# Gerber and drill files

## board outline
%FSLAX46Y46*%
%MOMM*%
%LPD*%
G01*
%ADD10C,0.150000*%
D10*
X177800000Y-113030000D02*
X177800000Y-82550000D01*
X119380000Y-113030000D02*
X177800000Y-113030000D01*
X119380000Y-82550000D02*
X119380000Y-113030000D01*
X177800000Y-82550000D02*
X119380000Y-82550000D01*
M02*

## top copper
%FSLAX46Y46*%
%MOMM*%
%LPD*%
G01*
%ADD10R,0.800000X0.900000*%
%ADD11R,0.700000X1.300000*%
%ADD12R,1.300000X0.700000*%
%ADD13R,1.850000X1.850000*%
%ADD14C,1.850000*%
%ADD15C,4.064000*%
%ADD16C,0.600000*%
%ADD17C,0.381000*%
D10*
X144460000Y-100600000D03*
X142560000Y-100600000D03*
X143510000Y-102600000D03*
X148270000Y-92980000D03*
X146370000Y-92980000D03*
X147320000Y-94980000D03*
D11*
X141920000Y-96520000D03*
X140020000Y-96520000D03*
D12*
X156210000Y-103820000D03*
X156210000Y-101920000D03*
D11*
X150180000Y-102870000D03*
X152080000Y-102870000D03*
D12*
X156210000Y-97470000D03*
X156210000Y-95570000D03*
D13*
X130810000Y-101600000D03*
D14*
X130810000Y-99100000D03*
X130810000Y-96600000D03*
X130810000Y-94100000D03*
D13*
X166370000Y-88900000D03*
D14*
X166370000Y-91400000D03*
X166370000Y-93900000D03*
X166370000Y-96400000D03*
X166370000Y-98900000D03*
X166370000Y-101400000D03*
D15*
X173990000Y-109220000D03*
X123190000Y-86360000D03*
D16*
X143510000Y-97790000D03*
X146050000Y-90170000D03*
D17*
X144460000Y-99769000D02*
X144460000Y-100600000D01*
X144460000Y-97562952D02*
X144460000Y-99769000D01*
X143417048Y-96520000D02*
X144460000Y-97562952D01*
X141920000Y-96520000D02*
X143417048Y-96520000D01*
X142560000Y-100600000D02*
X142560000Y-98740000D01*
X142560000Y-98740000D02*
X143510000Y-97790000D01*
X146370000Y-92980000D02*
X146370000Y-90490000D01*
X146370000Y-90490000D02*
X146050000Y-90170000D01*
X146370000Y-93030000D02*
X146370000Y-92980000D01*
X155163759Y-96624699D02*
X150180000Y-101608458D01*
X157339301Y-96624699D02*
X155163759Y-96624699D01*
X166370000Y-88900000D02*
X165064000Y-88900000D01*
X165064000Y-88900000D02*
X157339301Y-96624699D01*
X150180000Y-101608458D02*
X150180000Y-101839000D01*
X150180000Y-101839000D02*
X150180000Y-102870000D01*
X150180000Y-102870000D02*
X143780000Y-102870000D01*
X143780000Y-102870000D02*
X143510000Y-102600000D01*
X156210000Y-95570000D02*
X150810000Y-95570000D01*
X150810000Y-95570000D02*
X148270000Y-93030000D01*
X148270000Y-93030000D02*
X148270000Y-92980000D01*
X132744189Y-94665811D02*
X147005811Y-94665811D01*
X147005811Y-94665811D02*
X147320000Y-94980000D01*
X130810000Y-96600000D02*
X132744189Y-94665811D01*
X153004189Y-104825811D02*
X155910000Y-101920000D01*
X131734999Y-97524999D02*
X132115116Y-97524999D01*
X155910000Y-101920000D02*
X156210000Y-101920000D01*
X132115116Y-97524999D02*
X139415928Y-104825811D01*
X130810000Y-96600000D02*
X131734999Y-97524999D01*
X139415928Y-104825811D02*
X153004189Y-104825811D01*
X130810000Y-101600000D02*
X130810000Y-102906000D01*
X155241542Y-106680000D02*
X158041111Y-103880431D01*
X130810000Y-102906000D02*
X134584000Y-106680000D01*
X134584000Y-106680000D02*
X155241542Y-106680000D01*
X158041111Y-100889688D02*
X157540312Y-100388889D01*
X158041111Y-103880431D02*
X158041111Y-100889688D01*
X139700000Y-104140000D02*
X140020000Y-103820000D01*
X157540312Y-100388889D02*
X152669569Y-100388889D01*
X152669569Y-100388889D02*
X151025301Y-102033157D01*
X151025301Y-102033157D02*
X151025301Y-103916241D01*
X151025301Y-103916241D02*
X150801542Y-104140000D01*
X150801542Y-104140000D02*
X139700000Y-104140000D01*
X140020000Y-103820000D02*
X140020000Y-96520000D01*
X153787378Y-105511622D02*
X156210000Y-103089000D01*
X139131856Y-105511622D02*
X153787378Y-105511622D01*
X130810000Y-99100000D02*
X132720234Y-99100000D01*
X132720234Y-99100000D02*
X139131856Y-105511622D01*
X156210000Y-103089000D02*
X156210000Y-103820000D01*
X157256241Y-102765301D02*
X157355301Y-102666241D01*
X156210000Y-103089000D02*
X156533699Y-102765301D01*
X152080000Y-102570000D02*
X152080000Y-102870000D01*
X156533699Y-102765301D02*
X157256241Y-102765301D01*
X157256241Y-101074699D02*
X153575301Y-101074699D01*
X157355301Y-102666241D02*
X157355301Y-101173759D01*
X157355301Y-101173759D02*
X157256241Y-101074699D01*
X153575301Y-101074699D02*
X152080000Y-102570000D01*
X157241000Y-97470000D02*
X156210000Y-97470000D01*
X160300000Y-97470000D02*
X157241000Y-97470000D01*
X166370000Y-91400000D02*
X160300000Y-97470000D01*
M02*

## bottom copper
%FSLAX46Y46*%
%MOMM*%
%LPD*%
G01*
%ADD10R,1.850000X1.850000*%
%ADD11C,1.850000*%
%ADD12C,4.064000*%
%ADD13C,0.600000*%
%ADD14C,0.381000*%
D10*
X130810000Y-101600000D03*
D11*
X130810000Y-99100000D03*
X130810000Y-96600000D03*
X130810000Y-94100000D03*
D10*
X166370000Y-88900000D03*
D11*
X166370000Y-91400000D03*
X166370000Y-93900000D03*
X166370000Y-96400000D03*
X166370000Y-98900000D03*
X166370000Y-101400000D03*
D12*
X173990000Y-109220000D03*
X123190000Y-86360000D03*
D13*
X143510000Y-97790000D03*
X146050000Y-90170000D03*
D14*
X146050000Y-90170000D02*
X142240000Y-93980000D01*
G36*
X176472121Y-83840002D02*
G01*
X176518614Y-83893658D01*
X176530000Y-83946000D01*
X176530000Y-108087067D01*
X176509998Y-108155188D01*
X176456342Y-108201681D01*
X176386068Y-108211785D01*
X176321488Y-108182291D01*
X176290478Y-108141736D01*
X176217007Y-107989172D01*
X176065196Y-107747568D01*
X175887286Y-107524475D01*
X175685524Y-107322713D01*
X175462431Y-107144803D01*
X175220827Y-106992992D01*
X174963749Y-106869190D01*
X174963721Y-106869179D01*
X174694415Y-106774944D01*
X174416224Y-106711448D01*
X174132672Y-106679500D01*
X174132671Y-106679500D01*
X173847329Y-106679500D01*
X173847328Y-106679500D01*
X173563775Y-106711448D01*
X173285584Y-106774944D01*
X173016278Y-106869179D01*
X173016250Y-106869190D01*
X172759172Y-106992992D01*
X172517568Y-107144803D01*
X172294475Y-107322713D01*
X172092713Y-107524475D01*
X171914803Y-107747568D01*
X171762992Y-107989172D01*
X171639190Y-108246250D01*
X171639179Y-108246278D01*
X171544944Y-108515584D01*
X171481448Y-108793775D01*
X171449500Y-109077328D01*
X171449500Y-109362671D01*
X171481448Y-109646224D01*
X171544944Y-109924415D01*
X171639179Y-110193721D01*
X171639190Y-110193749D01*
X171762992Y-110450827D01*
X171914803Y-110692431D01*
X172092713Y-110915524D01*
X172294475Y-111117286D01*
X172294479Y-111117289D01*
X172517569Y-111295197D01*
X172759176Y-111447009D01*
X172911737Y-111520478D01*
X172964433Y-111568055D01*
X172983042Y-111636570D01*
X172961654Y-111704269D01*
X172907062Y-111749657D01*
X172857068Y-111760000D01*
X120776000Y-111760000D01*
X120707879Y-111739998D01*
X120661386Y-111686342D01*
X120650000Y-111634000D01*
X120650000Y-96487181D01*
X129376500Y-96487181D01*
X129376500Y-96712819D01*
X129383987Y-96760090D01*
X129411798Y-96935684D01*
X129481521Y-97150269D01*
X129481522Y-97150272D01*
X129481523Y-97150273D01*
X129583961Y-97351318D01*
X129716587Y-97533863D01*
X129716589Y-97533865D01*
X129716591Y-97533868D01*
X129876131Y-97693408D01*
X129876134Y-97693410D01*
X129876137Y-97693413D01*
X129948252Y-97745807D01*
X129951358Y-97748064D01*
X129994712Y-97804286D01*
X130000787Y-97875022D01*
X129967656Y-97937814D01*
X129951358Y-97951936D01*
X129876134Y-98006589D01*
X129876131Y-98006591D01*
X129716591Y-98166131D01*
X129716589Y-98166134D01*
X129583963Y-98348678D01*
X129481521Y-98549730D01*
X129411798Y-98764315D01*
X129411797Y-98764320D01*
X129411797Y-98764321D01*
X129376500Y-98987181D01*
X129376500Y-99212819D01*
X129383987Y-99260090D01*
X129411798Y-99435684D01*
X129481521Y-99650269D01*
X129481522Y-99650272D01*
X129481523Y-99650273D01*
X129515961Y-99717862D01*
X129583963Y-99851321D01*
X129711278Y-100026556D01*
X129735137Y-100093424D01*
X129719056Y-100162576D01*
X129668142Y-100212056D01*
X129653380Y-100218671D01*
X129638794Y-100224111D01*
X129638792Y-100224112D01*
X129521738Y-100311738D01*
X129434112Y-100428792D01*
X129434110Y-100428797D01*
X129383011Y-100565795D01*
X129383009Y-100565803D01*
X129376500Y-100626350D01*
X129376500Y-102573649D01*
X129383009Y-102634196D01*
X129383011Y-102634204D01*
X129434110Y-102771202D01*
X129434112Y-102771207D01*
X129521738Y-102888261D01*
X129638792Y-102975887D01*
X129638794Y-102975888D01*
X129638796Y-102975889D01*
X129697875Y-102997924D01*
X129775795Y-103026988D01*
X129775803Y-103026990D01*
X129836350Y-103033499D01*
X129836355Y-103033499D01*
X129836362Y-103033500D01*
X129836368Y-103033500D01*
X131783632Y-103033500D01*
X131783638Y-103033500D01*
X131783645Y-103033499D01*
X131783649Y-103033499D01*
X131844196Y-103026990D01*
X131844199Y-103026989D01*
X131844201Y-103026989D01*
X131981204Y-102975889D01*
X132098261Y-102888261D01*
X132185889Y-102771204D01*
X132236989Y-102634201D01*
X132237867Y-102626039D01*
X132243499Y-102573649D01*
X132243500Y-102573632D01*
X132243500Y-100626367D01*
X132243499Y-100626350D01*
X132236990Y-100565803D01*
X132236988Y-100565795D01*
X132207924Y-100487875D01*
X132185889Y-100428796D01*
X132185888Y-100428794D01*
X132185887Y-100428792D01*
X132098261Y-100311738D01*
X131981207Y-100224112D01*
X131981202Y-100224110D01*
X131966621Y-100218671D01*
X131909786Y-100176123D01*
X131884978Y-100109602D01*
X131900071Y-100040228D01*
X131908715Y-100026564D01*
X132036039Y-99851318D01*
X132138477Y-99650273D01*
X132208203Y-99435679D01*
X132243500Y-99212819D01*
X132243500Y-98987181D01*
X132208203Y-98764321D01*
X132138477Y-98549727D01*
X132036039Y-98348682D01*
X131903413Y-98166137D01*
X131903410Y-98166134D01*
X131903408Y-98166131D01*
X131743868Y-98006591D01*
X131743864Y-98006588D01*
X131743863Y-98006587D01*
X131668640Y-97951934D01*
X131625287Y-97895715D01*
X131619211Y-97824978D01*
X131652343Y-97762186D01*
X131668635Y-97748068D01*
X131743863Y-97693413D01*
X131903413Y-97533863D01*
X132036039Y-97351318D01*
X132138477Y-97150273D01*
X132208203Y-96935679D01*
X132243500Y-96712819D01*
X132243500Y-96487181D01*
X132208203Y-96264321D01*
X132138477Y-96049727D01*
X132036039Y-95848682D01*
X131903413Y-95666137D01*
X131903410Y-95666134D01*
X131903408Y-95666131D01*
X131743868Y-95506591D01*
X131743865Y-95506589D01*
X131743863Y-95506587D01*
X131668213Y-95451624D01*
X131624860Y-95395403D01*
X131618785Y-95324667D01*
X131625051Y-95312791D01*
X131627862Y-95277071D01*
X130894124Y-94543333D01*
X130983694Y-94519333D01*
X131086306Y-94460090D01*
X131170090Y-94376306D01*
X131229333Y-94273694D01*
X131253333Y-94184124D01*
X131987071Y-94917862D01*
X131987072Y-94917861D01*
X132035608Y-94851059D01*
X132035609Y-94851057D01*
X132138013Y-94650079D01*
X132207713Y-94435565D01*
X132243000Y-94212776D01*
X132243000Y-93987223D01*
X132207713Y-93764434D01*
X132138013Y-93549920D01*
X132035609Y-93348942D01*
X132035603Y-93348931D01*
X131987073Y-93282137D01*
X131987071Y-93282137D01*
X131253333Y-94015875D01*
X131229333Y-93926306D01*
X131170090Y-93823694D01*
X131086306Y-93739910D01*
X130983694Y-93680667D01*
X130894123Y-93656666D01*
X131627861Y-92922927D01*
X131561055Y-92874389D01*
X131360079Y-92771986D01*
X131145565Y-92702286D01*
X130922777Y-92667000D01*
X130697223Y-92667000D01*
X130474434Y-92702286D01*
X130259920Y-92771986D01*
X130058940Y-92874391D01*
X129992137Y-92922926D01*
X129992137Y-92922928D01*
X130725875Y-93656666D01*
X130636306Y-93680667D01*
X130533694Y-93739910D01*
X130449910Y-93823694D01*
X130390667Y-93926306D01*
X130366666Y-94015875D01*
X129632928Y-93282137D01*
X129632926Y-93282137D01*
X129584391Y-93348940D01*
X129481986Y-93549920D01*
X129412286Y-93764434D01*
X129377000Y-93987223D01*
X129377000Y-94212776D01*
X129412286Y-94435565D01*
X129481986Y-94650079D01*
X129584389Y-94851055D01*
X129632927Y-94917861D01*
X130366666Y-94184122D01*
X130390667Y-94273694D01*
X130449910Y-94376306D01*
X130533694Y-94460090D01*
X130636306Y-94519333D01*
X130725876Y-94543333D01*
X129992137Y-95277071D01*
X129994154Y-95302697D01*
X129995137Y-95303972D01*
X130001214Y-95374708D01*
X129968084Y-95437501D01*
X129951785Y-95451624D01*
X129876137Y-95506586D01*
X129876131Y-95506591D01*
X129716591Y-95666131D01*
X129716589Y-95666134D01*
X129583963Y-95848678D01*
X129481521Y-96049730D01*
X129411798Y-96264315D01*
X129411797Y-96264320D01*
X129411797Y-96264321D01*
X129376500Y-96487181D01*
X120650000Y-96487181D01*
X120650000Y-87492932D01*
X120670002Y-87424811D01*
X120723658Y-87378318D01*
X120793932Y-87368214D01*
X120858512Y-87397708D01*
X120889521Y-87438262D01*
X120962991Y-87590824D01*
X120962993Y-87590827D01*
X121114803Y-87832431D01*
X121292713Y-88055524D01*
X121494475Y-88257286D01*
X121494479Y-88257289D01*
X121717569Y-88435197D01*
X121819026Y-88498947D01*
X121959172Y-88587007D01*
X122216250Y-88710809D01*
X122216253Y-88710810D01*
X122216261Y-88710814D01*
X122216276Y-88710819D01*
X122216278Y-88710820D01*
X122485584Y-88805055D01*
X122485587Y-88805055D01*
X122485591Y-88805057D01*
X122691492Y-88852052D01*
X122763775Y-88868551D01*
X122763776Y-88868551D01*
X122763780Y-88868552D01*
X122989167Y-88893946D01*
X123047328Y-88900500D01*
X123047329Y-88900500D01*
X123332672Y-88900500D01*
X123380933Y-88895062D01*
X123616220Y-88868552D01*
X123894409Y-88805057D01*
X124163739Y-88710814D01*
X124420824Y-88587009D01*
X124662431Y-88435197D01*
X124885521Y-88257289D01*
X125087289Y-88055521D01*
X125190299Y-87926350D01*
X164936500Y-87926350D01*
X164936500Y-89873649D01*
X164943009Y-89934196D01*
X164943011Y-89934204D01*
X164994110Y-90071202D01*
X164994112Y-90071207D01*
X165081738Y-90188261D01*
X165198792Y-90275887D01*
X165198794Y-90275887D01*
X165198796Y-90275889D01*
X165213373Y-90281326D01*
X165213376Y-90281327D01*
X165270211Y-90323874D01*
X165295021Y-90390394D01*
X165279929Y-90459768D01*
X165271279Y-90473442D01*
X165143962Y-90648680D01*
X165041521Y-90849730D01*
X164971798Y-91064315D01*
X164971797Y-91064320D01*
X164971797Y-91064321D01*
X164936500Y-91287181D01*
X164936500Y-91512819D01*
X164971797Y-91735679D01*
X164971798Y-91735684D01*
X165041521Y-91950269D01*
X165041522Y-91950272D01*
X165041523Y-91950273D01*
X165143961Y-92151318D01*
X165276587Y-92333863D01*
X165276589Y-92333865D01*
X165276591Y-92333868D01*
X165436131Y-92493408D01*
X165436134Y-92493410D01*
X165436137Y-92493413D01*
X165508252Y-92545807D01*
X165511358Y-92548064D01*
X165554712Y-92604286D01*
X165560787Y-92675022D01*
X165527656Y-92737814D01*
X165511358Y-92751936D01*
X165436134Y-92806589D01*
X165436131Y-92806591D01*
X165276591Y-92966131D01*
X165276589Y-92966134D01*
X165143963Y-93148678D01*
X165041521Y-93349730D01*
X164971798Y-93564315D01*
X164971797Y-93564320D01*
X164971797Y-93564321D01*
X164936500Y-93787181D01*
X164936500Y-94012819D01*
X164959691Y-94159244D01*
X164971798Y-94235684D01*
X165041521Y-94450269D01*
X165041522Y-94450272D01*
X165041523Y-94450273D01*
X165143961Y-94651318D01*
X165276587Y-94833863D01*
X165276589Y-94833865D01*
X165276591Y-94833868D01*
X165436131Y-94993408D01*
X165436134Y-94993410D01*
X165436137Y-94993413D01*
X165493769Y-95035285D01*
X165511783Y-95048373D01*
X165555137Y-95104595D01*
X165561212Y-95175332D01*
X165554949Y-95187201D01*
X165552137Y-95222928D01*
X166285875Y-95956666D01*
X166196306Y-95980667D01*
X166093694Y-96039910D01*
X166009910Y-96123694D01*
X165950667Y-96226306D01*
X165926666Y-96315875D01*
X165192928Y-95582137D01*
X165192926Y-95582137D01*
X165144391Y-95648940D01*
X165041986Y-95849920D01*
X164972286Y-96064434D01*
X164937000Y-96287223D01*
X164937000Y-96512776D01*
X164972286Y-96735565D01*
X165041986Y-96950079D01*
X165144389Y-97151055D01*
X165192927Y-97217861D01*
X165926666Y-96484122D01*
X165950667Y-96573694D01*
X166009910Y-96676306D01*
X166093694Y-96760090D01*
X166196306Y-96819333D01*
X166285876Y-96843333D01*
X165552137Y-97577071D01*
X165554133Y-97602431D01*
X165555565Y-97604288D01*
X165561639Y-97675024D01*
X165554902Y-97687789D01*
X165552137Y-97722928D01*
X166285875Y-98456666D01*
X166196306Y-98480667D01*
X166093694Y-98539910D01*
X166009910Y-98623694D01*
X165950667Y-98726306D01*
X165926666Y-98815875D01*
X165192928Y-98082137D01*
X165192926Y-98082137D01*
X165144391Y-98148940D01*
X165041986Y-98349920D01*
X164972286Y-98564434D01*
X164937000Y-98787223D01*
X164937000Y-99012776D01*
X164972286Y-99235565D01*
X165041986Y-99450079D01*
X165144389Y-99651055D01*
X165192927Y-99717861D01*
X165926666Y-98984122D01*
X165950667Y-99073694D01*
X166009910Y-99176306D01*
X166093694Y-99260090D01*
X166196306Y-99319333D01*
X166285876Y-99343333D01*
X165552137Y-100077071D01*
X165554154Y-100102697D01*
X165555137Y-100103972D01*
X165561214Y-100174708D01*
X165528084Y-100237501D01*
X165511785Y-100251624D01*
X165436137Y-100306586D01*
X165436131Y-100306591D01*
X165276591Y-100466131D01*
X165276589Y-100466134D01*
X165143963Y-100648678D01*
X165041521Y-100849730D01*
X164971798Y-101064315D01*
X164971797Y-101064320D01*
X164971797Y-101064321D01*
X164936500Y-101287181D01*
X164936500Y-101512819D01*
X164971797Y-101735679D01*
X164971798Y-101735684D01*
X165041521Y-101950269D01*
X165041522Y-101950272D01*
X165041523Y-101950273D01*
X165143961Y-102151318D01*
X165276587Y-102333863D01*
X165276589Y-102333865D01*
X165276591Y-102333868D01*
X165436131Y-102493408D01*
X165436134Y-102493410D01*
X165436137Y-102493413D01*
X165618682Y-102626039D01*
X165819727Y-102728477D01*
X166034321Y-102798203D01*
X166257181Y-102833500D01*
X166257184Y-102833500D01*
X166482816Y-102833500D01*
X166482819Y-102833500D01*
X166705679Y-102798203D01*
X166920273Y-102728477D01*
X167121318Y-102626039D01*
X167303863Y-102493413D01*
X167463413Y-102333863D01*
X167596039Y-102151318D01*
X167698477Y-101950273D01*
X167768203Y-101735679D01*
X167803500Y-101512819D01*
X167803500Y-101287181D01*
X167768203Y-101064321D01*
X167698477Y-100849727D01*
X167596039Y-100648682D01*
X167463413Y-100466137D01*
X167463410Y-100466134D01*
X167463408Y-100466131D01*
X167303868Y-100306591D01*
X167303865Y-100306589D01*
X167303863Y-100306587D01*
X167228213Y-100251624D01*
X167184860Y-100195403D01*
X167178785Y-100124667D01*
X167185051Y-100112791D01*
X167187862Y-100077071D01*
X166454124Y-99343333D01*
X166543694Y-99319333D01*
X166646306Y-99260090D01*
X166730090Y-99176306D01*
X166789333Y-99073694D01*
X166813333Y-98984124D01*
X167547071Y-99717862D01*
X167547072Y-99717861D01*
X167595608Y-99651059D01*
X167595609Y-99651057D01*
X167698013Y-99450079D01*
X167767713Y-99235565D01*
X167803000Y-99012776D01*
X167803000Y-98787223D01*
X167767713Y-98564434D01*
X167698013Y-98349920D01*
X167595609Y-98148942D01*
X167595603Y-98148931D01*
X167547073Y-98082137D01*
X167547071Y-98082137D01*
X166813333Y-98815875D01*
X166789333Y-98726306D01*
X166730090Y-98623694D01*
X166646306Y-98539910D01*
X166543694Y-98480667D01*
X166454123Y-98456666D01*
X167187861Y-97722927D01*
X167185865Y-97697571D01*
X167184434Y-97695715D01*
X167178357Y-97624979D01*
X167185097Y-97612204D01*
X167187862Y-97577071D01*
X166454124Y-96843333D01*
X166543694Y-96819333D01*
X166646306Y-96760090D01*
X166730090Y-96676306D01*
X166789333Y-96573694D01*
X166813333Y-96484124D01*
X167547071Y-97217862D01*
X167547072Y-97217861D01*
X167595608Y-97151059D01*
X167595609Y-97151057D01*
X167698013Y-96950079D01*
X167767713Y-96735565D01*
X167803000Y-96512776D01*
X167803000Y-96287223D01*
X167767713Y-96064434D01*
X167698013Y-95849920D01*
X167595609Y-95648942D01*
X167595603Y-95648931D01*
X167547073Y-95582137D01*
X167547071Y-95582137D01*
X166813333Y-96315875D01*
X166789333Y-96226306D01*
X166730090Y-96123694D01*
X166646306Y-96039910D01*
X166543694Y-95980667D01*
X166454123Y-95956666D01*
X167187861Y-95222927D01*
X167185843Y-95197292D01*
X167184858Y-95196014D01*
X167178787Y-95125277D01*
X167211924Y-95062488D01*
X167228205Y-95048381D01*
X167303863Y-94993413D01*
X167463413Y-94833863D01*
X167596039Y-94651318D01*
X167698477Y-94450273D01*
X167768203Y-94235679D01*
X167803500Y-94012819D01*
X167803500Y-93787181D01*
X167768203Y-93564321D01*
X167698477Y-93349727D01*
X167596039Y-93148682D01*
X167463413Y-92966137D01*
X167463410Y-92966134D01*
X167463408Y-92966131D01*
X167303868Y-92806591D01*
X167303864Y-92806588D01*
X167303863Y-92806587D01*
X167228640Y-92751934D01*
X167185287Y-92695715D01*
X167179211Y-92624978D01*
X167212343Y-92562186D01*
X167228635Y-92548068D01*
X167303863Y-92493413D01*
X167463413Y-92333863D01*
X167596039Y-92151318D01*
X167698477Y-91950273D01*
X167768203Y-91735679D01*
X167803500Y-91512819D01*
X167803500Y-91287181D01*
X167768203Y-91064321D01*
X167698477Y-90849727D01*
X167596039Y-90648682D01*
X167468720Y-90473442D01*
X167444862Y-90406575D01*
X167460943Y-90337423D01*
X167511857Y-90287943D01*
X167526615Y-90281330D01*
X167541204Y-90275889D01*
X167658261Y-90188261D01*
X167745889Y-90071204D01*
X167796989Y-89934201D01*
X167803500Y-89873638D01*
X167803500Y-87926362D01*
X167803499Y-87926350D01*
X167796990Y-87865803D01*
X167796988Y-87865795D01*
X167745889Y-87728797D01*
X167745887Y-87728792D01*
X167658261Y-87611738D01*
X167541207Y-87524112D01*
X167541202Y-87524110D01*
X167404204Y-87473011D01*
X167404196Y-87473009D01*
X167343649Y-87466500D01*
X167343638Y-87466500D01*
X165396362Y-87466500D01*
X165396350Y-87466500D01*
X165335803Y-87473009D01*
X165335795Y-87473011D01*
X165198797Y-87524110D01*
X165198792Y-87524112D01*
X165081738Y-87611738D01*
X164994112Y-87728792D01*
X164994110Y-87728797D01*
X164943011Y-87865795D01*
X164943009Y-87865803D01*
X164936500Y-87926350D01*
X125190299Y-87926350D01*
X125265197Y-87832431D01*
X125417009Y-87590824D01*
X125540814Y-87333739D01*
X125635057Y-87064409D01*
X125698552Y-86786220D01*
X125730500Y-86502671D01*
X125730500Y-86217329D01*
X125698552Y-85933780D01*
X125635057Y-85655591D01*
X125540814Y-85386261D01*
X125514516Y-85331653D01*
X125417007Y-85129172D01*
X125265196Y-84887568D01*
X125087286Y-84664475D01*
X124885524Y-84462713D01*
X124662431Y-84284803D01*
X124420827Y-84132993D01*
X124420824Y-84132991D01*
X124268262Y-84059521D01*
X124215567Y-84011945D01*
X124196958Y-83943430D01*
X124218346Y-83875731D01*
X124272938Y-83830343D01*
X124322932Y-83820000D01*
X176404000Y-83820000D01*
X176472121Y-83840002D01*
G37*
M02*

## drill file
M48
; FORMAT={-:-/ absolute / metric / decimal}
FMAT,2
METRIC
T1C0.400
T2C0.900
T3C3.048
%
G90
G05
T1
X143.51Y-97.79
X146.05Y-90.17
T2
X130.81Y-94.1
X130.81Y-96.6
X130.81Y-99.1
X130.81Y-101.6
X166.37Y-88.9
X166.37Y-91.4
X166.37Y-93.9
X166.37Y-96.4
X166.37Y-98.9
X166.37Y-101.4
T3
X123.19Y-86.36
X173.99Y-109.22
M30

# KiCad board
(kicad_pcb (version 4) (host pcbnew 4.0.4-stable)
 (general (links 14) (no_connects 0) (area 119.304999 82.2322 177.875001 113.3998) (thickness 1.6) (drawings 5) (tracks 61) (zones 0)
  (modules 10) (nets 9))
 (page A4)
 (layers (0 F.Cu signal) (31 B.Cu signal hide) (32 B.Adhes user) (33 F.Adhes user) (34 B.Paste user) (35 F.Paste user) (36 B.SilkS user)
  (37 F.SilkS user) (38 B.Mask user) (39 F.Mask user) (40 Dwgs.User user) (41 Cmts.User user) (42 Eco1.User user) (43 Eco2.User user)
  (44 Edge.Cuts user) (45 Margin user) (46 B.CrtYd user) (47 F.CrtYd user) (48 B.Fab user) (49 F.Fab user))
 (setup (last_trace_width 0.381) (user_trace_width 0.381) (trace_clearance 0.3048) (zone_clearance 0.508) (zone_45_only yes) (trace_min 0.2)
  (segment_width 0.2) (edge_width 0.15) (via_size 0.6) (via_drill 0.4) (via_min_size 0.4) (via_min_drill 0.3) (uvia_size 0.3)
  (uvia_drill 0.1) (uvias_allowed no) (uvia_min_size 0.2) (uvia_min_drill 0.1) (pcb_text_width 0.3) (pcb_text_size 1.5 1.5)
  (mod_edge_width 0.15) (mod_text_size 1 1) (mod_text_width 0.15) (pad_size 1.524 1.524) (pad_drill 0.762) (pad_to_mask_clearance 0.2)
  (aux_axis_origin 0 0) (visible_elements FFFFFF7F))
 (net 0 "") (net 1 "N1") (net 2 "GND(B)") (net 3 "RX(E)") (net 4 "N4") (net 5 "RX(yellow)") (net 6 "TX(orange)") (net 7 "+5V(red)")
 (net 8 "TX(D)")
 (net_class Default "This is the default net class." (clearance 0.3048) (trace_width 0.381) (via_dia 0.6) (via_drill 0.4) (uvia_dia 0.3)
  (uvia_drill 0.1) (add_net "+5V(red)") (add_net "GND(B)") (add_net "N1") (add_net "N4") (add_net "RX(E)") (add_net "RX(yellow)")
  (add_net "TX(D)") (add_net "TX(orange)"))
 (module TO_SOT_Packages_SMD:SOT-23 (layer F.Cu) (at 143.51 101.6 270)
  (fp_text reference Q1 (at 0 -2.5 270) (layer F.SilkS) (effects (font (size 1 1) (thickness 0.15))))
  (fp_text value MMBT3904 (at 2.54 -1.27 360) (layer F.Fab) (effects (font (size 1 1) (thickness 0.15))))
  (pad 1 smd rect (at -1 -0.95 270) (size 0.9 0.8) (layers F.Cu F.Paste F.Mask) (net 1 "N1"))
  (pad 2 smd rect (at -1 0.95 270) (size 0.9 0.8) (layers F.Cu F.Paste F.Mask) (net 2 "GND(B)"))
  (pad 3 smd rect (at 1 0 270) (size 0.9 0.8) (layers F.Cu F.Paste F.Mask) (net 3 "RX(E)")))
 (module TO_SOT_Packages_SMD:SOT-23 (layer F.Cu) (at 147.32 93.98 270)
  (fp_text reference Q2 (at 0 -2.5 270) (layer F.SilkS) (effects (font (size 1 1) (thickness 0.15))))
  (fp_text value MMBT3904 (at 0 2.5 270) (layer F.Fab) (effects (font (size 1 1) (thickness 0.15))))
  (pad 1 smd rect (at -1 -0.95 270) (size 0.9 0.8) (layers F.Cu F.Paste F.Mask) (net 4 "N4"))
  (pad 2 smd rect (at -1 0.95 270) (size 0.9 0.8) (layers F.Cu F.Paste F.Mask) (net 2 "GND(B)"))
  (pad 3 smd rect (at 1 0 270) (size 0.9 0.8) (layers F.Cu F.Paste F.Mask) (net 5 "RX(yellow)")))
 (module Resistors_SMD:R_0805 (layer F.Cu) (at 140.97 96.52 180)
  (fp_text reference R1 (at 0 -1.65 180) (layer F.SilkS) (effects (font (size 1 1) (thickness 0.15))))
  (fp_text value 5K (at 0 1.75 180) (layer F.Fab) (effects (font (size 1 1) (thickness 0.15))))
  (pad 1 smd rect (at -0.95 0 180) (size 0.7 1.3) (layers F.Cu F.Paste F.Mask) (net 1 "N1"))
  (pad 2 smd rect (at 0.95 0 180) (size 0.7 1.3) (layers F.Cu F.Paste F.Mask) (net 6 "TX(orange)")))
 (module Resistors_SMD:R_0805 (layer F.Cu) (at 156.21 102.87 90)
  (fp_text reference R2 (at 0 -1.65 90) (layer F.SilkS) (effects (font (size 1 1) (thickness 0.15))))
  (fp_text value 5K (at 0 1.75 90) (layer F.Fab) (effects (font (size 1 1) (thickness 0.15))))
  (pad 1 smd rect (at -0.95 0 90) (size 0.7 1.3) (layers F.Cu F.Paste F.Mask) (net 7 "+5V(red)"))
  (pad 2 smd rect (at 0.95 0 90) (size 0.7 1.3) (layers F.Cu F.Paste F.Mask) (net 5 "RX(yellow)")))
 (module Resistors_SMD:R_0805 (layer F.Cu) (at 151.13 102.87)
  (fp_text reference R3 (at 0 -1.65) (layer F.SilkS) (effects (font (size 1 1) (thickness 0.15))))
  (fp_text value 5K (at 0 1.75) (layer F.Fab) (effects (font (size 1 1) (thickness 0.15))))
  (pad 1 smd rect (at -0.95 0) (size 0.7 1.3) (layers F.Cu F.Paste F.Mask) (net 3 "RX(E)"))
  (pad 2 smd rect (at 0.95 0) (size 0.7 1.3) (layers F.Cu F.Paste F.Mask) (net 7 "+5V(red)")))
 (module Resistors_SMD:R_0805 (layer F.Cu) (at 156.21 96.52 90)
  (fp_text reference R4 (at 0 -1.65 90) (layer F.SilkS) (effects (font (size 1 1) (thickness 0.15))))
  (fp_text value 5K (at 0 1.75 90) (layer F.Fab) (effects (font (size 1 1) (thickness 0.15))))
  (pad 1 smd rect (at -0.95 0 90) (size 0.7 1.3) (layers F.Cu F.Paste F.Mask) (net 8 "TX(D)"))
  (pad 2 smd rect (at 0.95 0 90) (size 0.7 1.3) (layers F.Cu F.Paste F.Mask) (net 4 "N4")))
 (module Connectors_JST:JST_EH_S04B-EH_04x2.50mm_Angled (layer F.Cu) (at 130.81 101.6 90)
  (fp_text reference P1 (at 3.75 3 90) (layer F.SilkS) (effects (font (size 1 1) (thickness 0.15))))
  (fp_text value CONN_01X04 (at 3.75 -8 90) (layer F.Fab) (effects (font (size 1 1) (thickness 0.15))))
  (pad 1 thru_hole rect (at 0 0 90) (size 1.85 1.85) (drill 0.9) (layers *.Cu *.Mask) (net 6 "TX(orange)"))
  (pad 2 thru_hole circle (at 2.5 0 90) (size 1.85 1.85) (drill 0.9) (layers *.Cu *.Mask) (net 7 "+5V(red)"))
  (pad 3 thru_hole circle (at 5 0 90) (size 1.85 1.85) (drill 0.9) (layers *.Cu *.Mask) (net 5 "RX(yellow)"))
  (pad 4 thru_hole circle (at 7.5 0 90) (size 1.85 1.85) (drill 0.9) (layers *.Cu *.Mask) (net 2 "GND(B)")))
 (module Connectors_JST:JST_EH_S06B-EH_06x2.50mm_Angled (layer F.Cu) (at 166.37 88.9 270)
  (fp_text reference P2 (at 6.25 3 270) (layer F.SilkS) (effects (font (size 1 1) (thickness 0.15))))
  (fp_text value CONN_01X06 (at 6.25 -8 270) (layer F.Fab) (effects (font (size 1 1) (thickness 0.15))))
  (pad 1 thru_hole rect (at 0 0 270) (size 1.85 1.85) (drill 0.9) (layers *.Cu *.Mask) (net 3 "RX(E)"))
  (pad 2 thru_hole circle (at 2.5 0 270) (size 1.85 1.85) (drill 0.9) (layers *.Cu *.Mask) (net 8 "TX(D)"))
  (pad 3 thru_hole circle (at 5 0 270) (size 1.85 1.85) (drill 0.9) (layers *.Cu *.Mask))
  (pad 4 thru_hole circle (at 7.5 0 270) (size 1.85 1.85) (drill 0.9) (layers *.Cu *.Mask) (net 2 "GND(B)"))
  (pad 5 thru_hole circle (at 10 0 270) (size 1.85 1.85) (drill 0.9) (layers *.Cu *.Mask) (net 2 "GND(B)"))
  (pad 6 thru_hole circle (at 12.5 0 270) (size 1.85 1.85) (drill 0.9) (layers *.Cu *.Mask)))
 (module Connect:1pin (layer F.Cu) (at 173.99 109.22)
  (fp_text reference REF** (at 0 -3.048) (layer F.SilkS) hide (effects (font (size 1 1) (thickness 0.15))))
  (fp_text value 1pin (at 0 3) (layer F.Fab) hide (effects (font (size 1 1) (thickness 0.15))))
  (pad 1 thru_hole circle (at 0 0) (size 4.064 4.064) (drill 3.048) (layers *.Cu *.Mask)))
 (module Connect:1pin (layer F.Cu) (at 123.19 86.36)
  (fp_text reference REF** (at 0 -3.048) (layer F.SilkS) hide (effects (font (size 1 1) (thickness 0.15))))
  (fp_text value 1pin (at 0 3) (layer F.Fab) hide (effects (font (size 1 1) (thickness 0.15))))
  (pad 1 thru_hole circle (at 0 0) (size 4.064 4.064) (drill 3.048) (layers *.Cu *.Mask)))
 (gr_line (start 177.8 113.03) (end 177.8 82.55) (angle 90) (layer Edge.Cuts) (width 0.15))
 (gr_line (start 119.38 113.03) (end 177.8 113.03) (angle 90) (layer Edge.Cuts) (width 0.15))
 (gr_line (start 119.38 82.55) (end 119.38 113.03) (angle 90) (layer Edge.Cuts) (width 0.15))
 (gr_line (start 177.8 82.55) (end 119.38 82.55) (angle 90) (layer Edge.Cuts) (width 0.15))
 (segment (start 144.46 99.769) (end 144.46 100.6) (width 0.381) (layer F.Cu) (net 1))
 (segment (start 144.46 97.562952) (end 144.46 99.769) (width 0.381) (layer F.Cu) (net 1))
 (segment (start 143.417048 96.52) (end 144.46 97.562952) (width 0.381) (layer F.Cu) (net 1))
 (segment (start 141.92 96.52) (end 143.417048 96.52) (width 0.381) (layer F.Cu) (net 1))
 (segment (start 142.56 100.6) (end 142.56 98.74) (width 0.381) (layer F.Cu) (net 2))
 (segment (start 142.56 98.74) (end 143.51 97.79) (width 0.381) (layer F.Cu) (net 2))
 (via (at 143.51 97.79) (size 0.6) (drill 0.4) (layers F.Cu B.Cu) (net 2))
 (segment (start 146.05 90.17) (end 142.24 93.98) (width 0.381) (layer B.Cu) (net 2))
 (segment (start 146.37 92.98) (end 146.37 90.49) (width 0.381) (layer F.Cu) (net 2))
 (segment (start 146.37 90.49) (end 146.05 90.17) (width 0.381) (layer F.Cu) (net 2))
 (via (at 146.05 90.17) (size 0.6) (drill 0.4) (layers F.Cu B.Cu) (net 2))
 (segment (start 146.37 93.03) (end 146.37 92.98) (width 0.381) (layer F.Cu) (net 2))
 (segment (start 155.163759 96.624699) (end 150.18 101.608458) (width 0.381) (layer F.Cu) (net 3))
 (segment (start 157.339301 96.624699) (end 155.163759 96.624699) (width 0.381) (layer F.Cu) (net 3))
 (segment (start 166.37 88.9) (end 165.064 88.9) (width 0.381) (layer F.Cu) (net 3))
 (segment (start 165.064 88.9) (end 157.339301 96.624699) (width 0.381) (layer F.Cu) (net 3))
 (segment (start 150.18 101.608458) (end 150.18 101.839) (width 0.381) (layer F.Cu) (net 3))
 (segment (start 150.18 101.839) (end 150.18 102.87) (width 0.381) (layer F.Cu) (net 3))
 (segment (start 150.18 102.87) (end 143.78 102.87) (width 0.381) (layer F.Cu) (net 3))
 (segment (start 143.78 102.87) (end 143.51 102.6) (width 0.381) (layer F.Cu) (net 3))
 (segment (start 156.21 95.57) (end 150.81 95.57) (width 0.381) (layer F.Cu) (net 4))
 (segment (start 150.81 95.57) (end 148.27 93.03) (width 0.381) (layer F.Cu) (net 4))
 (segment (start 148.27 93.03) (end 148.27 92.98) (width 0.381) (layer F.Cu) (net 4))
 (segment (start 132.744189 94.665811) (end 147.005811 94.665811) (width 0.381) (layer F.Cu) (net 5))
 (segment (start 147.005811 94.665811) (end 147.32 94.98) (width 0.381) (layer F.Cu) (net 5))
 (segment (start 130.81 96.6) (end 132.744189 94.665811) (width 0.381) (layer F.Cu) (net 5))
 (segment (start 153.004189 104.825811) (end 155.91 101.92) (width 0.381) (layer F.Cu) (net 5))
 (segment (start 131.734999 97.524999) (end 132.115116 97.524999) (width 0.381) (layer F.Cu) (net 5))
 (segment (start 155.91 101.92) (end 156.21 101.92) (width 0.381) (layer F.Cu) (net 5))
 (segment (start 132.115116 97.524999) (end 139.415928 104.825811) (width 0.381) (layer F.Cu) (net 5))
 (segment (start 130.81 96.6) (end 131.734999 97.524999) (width 0.381) (layer F.Cu) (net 5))
 (segment (start 139.415928 104.825811) (end 153.004189 104.825811) (width 0.381) (layer F.Cu) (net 5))
 (segment (start 130.81 101.6) (end 130.81 102.906) (width 0.381) (layer F.Cu) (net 6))
 (segment (start 155.241542 106.68) (end 158.041111 103.880431) (width 0.381) (layer F.Cu) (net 6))
 (segment (start 130.81 102.906) (end 134.584 106.68) (width 0.381) (layer F.Cu) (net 6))
 (segment (start 134.584 106.68) (end 155.241542 106.68) (width 0.381) (layer F.Cu) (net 6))
 (segment (start 158.041111 100.889688) (end 157.540312 100.388889) (width 0.381) (layer F.Cu) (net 6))
 (segment (start 158.041111 103.880431) (end 158.041111 100.889688) (width 0.381) (layer F.Cu) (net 6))
 (segment (start 139.7 104.14) (end 140.02 103.82) (width 0.381) (layer F.Cu) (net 6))
 (segment (start 157.540312 100.388889) (end 152.669569 100.388889) (width 0.381) (layer F.Cu) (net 6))
 (segment (start 152.669569 100.388889) (end 151.025301 102.033157) (width 0.381) (layer F.Cu) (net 6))
 (segment (start 151.025301 102.033157) (end 151.025301 103.916241) (width 0.381) (layer F.Cu) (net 6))
 (segment (start 151.025301 103.916241) (end 150.801542 104.14) (width 0.381) (layer F.Cu) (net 6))
 (segment (start 150.801542 104.14) (end 139.7 104.14) (width 0.381) (layer F.Cu) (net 6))
 (segment (start 140.02 103.82) (end 140.02 96.52) (width 0.381) (layer F.Cu) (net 6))
 (segment (start 153.787378 105.511622) (end 156.21 103.089) (width 0.381) (layer F.Cu) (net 7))
 (segment (start 139.131856 105.511622) (end 153.787378 105.511622) (width 0.381) (layer F.Cu) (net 7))
 (segment (start 130.81 99.1) (end 132.720234 99.1) (width 0.381) (layer F.Cu) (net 7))
 (segment (start 132.720234 99.1) (end 139.131856 105.511622) (width 0.381) (layer F.Cu) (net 7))
 (segment (start 156.21 103.089) (end 156.21 103.82) (width 0.381) (layer F.Cu) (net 7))
 (segment (start 157.256241 102.765301) (end 157.355301 102.666241) (width 0.381) (layer F.Cu) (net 7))
 (segment (start 156.21 103.089) (end 156.533699 102.765301) (width 0.381) (layer F.Cu) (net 7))
 (segment (start 152.08 102.57) (end 152.08 102.87) (width 0.381) (layer F.Cu) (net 7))
 (segment (start 156.533699 102.765301) (end 157.256241 102.765301) (width 0.381) (layer F.Cu) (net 7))
 (segment (start 157.256241 101.074699) (end 153.575301 101.074699) (width 0.381) (layer F.Cu) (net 7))
 (segment (start 157.355301 102.666241) (end 157.355301 101.173759) (width 0.381) (layer F.Cu) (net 7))
 (segment (start 157.355301 101.173759) (end 157.256241 101.074699) (width 0.381) (layer F.Cu) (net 7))
 (segment (start 153.575301 101.074699) (end 152.08 102.57) (width 0.381) (layer F.Cu) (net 7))
 (segment (start 157.241 97.47) (end 156.21 97.47) (width 0.381) (layer F.Cu) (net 8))
 (segment (start 160.3 97.47) (end 157.241 97.47) (width 0.381) (layer F.Cu) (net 8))
 (segment (start 166.37 91.4) (end 160.3 97.47) (width 0.381) (layer F.Cu) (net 8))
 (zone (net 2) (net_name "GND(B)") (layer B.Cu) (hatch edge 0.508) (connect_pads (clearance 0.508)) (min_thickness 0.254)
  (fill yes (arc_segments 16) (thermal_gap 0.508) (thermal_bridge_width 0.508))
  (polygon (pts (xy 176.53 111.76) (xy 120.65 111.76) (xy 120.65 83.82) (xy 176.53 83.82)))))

